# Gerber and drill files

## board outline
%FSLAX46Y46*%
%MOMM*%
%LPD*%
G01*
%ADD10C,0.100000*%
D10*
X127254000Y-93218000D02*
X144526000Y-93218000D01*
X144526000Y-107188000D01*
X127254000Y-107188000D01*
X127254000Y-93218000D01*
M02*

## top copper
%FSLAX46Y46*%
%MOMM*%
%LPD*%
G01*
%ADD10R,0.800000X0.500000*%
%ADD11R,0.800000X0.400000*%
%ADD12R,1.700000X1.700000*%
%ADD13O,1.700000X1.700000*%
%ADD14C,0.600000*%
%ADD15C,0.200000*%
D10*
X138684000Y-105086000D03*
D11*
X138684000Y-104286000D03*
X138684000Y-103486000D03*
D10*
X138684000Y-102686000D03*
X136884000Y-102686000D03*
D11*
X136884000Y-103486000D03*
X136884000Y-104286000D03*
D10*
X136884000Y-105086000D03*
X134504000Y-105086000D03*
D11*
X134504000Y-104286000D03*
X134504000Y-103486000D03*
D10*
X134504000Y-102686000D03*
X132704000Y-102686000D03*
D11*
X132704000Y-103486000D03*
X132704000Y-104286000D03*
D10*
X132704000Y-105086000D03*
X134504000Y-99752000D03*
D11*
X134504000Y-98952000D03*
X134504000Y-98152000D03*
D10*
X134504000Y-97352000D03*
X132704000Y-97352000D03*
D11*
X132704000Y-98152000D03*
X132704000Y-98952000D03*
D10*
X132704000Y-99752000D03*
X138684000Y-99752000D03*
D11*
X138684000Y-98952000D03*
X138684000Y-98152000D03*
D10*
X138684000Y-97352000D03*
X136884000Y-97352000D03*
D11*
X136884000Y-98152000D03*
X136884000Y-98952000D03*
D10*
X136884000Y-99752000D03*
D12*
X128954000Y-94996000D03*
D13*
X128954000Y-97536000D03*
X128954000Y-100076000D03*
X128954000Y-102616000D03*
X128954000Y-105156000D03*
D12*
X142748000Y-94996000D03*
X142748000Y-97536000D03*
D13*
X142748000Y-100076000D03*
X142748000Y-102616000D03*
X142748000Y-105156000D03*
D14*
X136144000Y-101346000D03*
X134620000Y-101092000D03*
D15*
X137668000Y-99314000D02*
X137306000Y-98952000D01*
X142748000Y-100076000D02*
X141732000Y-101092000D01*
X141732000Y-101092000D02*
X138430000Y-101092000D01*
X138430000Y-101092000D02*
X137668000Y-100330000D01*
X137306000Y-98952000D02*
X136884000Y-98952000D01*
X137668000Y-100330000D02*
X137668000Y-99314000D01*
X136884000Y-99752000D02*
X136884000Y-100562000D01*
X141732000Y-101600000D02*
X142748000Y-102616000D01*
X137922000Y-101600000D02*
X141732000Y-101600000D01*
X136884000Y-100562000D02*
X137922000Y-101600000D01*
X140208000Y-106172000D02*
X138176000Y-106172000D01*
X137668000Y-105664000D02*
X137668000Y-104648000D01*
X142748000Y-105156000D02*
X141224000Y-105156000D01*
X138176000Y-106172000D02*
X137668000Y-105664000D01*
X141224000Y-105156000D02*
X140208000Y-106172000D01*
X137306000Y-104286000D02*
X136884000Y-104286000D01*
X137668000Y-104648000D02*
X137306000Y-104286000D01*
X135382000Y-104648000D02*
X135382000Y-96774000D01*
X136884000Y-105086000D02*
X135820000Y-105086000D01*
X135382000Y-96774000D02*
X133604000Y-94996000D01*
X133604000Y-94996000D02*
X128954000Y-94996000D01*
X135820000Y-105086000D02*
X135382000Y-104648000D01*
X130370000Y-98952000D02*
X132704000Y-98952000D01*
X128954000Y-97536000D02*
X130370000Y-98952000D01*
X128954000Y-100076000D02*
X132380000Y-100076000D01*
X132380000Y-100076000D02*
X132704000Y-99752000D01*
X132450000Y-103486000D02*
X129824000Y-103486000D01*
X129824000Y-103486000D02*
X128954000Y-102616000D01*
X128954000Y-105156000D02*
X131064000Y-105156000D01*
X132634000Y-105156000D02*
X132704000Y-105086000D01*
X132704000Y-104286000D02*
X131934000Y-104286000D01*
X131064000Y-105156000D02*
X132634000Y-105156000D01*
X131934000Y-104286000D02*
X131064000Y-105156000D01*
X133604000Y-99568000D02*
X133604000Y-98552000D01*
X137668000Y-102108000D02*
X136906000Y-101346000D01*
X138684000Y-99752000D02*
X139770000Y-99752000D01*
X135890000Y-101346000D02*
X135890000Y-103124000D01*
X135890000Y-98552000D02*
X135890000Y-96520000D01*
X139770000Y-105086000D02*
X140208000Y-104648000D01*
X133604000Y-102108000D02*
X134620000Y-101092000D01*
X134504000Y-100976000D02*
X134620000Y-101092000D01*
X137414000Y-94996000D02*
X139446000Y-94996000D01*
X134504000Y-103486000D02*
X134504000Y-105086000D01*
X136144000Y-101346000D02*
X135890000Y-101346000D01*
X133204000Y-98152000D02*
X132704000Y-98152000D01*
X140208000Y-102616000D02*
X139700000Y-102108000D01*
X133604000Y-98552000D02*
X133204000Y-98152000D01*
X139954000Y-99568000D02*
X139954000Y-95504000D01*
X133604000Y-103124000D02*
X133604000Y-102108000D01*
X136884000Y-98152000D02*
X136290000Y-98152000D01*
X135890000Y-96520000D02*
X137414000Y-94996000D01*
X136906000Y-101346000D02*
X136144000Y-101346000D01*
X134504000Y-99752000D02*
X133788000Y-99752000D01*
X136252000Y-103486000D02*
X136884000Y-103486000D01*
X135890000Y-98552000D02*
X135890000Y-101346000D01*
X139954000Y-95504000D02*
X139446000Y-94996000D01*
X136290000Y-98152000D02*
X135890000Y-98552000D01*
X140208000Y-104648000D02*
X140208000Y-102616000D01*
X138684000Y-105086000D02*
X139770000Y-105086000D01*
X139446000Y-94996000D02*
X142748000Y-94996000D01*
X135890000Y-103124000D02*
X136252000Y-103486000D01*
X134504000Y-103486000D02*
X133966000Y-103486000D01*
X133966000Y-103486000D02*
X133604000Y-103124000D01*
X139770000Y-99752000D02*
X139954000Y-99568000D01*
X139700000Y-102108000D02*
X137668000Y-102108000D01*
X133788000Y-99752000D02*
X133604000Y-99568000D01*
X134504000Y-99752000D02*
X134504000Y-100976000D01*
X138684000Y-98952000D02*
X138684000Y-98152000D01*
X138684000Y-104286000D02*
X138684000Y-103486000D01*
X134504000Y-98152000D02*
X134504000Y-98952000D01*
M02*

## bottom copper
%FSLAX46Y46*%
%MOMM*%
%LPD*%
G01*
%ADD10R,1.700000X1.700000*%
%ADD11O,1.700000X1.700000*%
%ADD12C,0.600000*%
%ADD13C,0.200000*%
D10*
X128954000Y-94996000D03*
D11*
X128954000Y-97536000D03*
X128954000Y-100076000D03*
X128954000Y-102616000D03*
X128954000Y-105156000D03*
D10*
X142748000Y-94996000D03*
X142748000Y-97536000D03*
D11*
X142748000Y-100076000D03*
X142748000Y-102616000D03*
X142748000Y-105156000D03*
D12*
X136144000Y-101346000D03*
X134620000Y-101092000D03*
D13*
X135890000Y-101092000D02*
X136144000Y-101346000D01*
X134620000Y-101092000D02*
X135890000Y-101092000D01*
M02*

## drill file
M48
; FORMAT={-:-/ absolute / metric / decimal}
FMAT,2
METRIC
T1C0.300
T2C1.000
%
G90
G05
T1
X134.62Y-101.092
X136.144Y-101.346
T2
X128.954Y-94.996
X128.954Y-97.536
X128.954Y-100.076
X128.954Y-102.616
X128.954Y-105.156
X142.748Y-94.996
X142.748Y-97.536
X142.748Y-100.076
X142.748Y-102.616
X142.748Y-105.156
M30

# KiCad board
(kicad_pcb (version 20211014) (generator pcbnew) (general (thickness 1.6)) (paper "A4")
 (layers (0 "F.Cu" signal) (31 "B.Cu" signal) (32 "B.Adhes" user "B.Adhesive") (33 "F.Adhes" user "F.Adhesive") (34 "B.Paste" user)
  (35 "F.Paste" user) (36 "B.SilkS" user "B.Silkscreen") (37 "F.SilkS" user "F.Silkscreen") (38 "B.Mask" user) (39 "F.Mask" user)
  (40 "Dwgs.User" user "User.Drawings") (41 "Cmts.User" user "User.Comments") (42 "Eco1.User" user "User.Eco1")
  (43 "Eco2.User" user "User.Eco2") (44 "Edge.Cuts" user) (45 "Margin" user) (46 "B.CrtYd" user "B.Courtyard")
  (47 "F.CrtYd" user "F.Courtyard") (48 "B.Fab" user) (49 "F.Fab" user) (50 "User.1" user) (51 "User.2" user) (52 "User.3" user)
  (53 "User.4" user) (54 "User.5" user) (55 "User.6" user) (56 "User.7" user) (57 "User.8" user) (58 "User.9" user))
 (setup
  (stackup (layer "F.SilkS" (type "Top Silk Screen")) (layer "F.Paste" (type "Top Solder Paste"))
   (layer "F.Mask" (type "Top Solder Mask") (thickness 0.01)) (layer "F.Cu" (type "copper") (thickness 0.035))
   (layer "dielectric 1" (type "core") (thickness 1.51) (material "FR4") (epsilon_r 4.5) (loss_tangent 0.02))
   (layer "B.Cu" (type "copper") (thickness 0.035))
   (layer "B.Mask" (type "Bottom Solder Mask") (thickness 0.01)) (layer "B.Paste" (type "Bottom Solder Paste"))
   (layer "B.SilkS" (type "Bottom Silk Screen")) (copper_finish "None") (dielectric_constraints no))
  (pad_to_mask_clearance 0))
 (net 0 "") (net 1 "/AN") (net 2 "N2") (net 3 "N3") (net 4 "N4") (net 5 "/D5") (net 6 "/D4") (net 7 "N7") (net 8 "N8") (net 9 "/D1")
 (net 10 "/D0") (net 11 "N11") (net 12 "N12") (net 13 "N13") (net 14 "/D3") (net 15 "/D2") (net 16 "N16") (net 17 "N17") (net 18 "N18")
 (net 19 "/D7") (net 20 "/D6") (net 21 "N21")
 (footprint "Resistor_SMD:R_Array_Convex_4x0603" (layer "F.Cu") (at 137.784 103.886 180)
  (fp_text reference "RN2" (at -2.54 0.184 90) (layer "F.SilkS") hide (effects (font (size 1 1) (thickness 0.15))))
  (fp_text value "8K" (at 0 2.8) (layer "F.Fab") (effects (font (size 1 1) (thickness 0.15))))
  (pad "1" smd rect (at -0.9 -1.2 180) (size 0.8 0.5) (layers "F.Cu" "F.Paste" "F.Mask") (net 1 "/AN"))
  (pad "2" smd rect (at -0.9 -0.4 180) (size 0.8 0.4) (layers "F.Cu" "F.Paste" "F.Mask") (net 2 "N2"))
  (pad "3" smd rect (at -0.9 0.4 180) (size 0.8 0.4) (layers "F.Cu" "F.Paste" "F.Mask") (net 2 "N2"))
  (pad "4" smd rect (at -0.9 1.2 180) (size 0.8 0.5) (layers "F.Cu" "F.Paste" "F.Mask") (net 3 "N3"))
  (pad "5" smd rect (at 0.9 1.2 180) (size 0.8 0.5) (layers "F.Cu" "F.Paste" "F.Mask") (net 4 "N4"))
  (pad "6" smd rect (at 0.9 0.4 180) (size 0.8 0.4) (layers "F.Cu" "F.Paste" "F.Mask") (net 1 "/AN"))
  (pad "7" smd rect (at 0.9 -0.4 180) (size 0.8 0.4) (layers "F.Cu" "F.Paste" "F.Mask") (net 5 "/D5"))
  (pad "8" smd rect (at 0.9 -1.2 180) (size 0.8 0.5) (layers "F.Cu" "F.Paste" "F.Mask") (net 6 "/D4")))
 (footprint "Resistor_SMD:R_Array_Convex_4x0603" (layer "F.Cu") (at 133.604 103.886 180)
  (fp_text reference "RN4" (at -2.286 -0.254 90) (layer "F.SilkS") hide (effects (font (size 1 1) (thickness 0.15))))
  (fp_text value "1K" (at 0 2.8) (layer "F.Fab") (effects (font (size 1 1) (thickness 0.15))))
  (pad "1" smd rect (at -0.9 -1.2 180) (size 0.8 0.5) (layers "F.Cu" "F.Paste" "F.Mask") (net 1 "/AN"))
  (pad "2" smd rect (at -0.9 -0.4 180) (size 0.8 0.4) (layers "F.Cu" "F.Paste" "F.Mask") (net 1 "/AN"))
  (pad "3" smd rect (at -0.9 0.4 180) (size 0.8 0.4) (layers "F.Cu" "F.Paste" "F.Mask") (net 1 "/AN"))
  (pad "4" smd rect (at -0.9 1.2 180) (size 0.8 0.5) (layers "F.Cu" "F.Paste" "F.Mask") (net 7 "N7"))
  (pad "5" smd rect (at 0.9 1.2 180) (size 0.8 0.5) (layers "F.Cu" "F.Paste" "F.Mask") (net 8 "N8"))
  (pad "6" smd rect (at 0.9 0.4 180) (size 0.8 0.4) (layers "F.Cu" "F.Paste" "F.Mask") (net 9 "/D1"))
  (pad "7" smd rect (at 0.9 -0.4 180) (size 0.8 0.4) (layers "F.Cu" "F.Paste" "F.Mask") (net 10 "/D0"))
  (pad "8" smd rect (at 0.9 -1.2 180) (size 0.8 0.5) (layers "F.Cu" "F.Paste" "F.Mask") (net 10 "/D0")))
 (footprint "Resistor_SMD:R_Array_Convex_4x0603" (layer "F.Cu") (at 133.604 98.552 180)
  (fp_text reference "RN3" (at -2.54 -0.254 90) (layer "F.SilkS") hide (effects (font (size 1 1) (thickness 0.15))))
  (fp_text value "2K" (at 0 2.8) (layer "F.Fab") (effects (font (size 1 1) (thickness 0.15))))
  (pad "1" smd rect (at -0.9 -1.2 180) (size 0.8 0.5) (layers "F.Cu" "F.Paste" "F.Mask") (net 1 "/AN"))
  (pad "2" smd rect (at -0.9 -0.4 180) (size 0.8 0.4) (layers "F.Cu" "F.Paste" "F.Mask") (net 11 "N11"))
  (pad "3" smd rect (at -0.9 0.4 180) (size 0.8 0.4) (layers "F.Cu" "F.Paste" "F.Mask") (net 11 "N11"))
  (pad "4" smd rect (at -0.9 1.2 180) (size 0.8 0.5) (layers "F.Cu" "F.Paste" "F.Mask") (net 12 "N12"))
  (pad "5" smd rect (at 0.9 1.2 180) (size 0.8 0.5) (layers "F.Cu" "F.Paste" "F.Mask") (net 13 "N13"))
  (pad "6" smd rect (at 0.9 0.4 180) (size 0.8 0.4) (layers "F.Cu" "F.Paste" "F.Mask") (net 1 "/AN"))
  (pad "7" smd rect (at 0.9 -0.4 180) (size 0.8 0.4) (layers "F.Cu" "F.Paste" "F.Mask") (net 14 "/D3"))
  (pad "8" smd rect (at 0.9 -1.2 180) (size 0.8 0.5) (layers "F.Cu" "F.Paste" "F.Mask") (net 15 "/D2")))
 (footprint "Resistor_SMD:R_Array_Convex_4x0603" (layer "F.Cu") (at 137.784 98.552 180)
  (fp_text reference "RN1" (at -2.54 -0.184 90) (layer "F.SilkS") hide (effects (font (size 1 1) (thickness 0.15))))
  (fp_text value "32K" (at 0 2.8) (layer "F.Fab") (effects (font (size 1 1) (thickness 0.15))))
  (pad "1" smd rect (at -0.9 -1.2 180) (size 0.8 0.5) (layers "F.Cu" "F.Paste" "F.Mask") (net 1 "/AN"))
  (pad "2" smd rect (at -0.9 -0.4 180) (size 0.8 0.4) (layers "F.Cu" "F.Paste" "F.Mask") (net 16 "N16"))
  (pad "3" smd rect (at -0.9 0.4 180) (size 0.8 0.4) (layers "F.Cu" "F.Paste" "F.Mask") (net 16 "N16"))
  (pad "4" smd rect (at -0.9 1.2 180) (size 0.8 0.5) (layers "F.Cu" "F.Paste" "F.Mask") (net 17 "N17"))
  (pad "5" smd rect (at 0.9 1.2 180) (size 0.8 0.5) (layers "F.Cu" "F.Paste" "F.Mask") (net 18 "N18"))
  (pad "6" smd rect (at 0.9 0.4 180) (size 0.8 0.4) (layers "F.Cu" "F.Paste" "F.Mask") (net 1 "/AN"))
  (pad "7" smd rect (at 0.9 -0.4 180) (size 0.8 0.4) (layers "F.Cu" "F.Paste" "F.Mask") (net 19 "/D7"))
  (pad "8" smd rect (at 0.9 -1.2 180) (size 0.8 0.5) (layers "F.Cu" "F.Paste" "F.Mask") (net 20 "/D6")))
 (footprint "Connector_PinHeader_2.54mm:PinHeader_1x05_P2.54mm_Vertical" (layer "B.Cu") (at 128.954 94.996 180)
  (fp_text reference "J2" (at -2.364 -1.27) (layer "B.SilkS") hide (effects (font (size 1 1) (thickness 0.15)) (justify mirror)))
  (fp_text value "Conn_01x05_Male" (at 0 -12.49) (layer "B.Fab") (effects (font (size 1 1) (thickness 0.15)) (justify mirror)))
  (pad "1" thru_hole rect (at 0 0 180) (size 1.7 1.7) (drill 1) (layers *.Cu *.Mask) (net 6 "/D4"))
  (pad "2" thru_hole oval (at 0 -2.54 180) (size 1.7 1.7) (drill 1) (layers *.Cu *.Mask) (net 14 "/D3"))
  (pad "3" thru_hole oval (at 0 -5.08 180) (size 1.7 1.7) (drill 1) (layers *.Cu *.Mask) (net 15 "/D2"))
  (pad "4" thru_hole oval (at 0 -7.62 180) (size 1.7 1.7) (drill 1) (layers *.Cu *.Mask) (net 9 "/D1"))
  (pad "5" thru_hole oval (at 0 -10.16 180) (size 1.7 1.7) (drill 1) (layers *.Cu *.Mask) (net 10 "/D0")))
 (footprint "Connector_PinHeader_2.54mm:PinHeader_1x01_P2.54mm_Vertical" (layer "B.Cu") (at 142.748 94.996 180)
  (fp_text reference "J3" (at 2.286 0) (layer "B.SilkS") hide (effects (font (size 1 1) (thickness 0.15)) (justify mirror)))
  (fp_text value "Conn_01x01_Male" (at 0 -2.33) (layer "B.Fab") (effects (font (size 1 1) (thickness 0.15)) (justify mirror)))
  (pad "1" thru_hole rect (at 0 0 180) (size 1.7 1.7) (drill 1) (layers *.Cu *.Mask) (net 1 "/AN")))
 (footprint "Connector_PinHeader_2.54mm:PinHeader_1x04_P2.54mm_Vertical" (layer "B.Cu") (at 142.748 97.536 180)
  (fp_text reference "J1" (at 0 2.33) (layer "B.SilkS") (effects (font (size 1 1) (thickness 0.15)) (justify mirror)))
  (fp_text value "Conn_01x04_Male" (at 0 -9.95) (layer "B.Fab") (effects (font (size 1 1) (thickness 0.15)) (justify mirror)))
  (pad "1" thru_hole rect (at 0 0 180) (size 1.7 1.7) (drill 1) (layers *.Cu *.Mask) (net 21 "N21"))
  (pad "2" thru_hole oval (at 0 -2.54 180) (size 1.7 1.7) (drill 1) (layers *.Cu *.Mask) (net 19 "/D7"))
  (pad "3" thru_hole oval (at 0 -5.08 180) (size 1.7 1.7) (drill 1) (layers *.Cu *.Mask) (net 20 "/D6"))
  (pad "4" thru_hole oval (at 0 -7.62 180) (size 1.7 1.7) (drill 1) (layers *.Cu *.Mask) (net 5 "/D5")))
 (gr_rect (start 127.254 93.218) (end 144.526 107.188) (layer "Edge.Cuts") (width 0.1) (fill none))
 (segment (start 137.668 99.314) (end 137.306 98.952) (width 0.2) (layer "F.Cu") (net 19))
 (segment (start 142.748 100.076) (end 141.732 101.092) (width 0.2) (layer "F.Cu") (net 19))
 (segment (start 141.732 101.092) (end 138.43 101.092) (width 0.2) (layer "F.Cu") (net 19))
 (segment (start 138.43 101.092) (end 137.668 100.33) (width 0.2) (layer "F.Cu") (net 19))
 (segment (start 137.306 98.952) (end 136.884 98.952) (width 0.2) (layer "F.Cu") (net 19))
 (segment (start 137.668 100.33) (end 137.668 99.314) (width 0.2) (layer "F.Cu") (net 19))
 (segment (start 136.884 99.752) (end 136.884 100.562) (width 0.2) (layer "F.Cu") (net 20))
 (segment (start 141.732 101.6) (end 142.748 102.616) (width 0.2) (layer "F.Cu") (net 20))
 (segment (start 137.922 101.6) (end 141.732 101.6) (width 0.2) (layer "F.Cu") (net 20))
 (segment (start 136.884 100.562) (end 137.922 101.6) (width 0.2) (layer "F.Cu") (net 20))
 (segment (start 140.208 106.172) (end 138.176 106.172) (width 0.2) (layer "F.Cu") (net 5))
 (segment (start 137.668 105.664) (end 137.668 104.648) (width 0.2) (layer "F.Cu") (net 5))
 (segment (start 142.748 105.156) (end 141.224 105.156) (width 0.2) (layer "F.Cu") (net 5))
 (segment (start 138.176 106.172) (end 137.668 105.664) (width 0.2) (layer "F.Cu") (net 5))
 (segment (start 141.224 105.156) (end 140.208 106.172) (width 0.2) (layer "F.Cu") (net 5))
 (segment (start 137.306 104.286) (end 136.884 104.286) (width 0.2) (layer "F.Cu") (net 5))
 (segment (start 137.668 104.648) (end 137.306 104.286) (width 0.2) (layer "F.Cu") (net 5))
 (segment (start 135.382 104.648) (end 135.382 96.774) (width 0.2) (layer "F.Cu") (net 6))
 (segment (start 136.884 105.086) (end 135.82 105.086) (width 0.2) (layer "F.Cu") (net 6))
 (segment (start 135.382 96.774) (end 133.604 94.996) (width 0.2) (layer "F.Cu") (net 6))
 (segment (start 133.604 94.996) (end 128.954 94.996) (width 0.2) (layer "F.Cu") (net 6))
 (segment (start 135.82 105.086) (end 135.382 104.648) (width 0.2) (layer "F.Cu") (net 6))
 (segment (start 130.37 98.952) (end 132.704 98.952) (width 0.2) (layer "F.Cu") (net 14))
 (segment (start 128.954 97.536) (end 130.37 98.952) (width 0.2) (layer "F.Cu") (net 14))
 (segment (start 128.954 100.076) (end 132.38 100.076) (width 0.2) (layer "F.Cu") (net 15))
 (segment (start 132.38 100.076) (end 132.704 99.752) (width 0.2) (layer "F.Cu") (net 15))
 (segment (start 132.45 103.486) (end 129.824 103.486) (width 0.2) (layer "F.Cu") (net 9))
 (segment (start 129.824 103.486) (end 128.954 102.616) (width 0.2) (layer "F.Cu") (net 9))
 (segment (start 128.954 105.156) (end 131.064 105.156) (width 0.2) (layer "F.Cu") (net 10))
 (segment (start 132.634 105.156) (end 132.704 105.086) (width 0.2) (layer "F.Cu") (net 10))
 (segment (start 132.704 104.286) (end 131.934 104.286) (width 0.2) (layer "F.Cu") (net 10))
 (segment (start 131.064 105.156) (end 132.634 105.156) (width 0.2) (layer "F.Cu") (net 10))
 (segment (start 131.934 104.286) (end 131.064 105.156) (width 0.2) (layer "F.Cu") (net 10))
 (segment (start 133.604 99.568) (end 133.604 98.552) (width 0.2) (layer "F.Cu") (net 1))
 (segment (start 137.668 102.108) (end 136.906 101.346) (width 0.2) (layer "F.Cu") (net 1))
 (segment (start 138.684 99.752) (end 139.77 99.752) (width 0.2) (layer "F.Cu") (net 1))
 (segment (start 135.89 101.346) (end 135.89 103.124) (width 0.2) (layer "F.Cu") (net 1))
 (segment (start 135.89 98.552) (end 135.89 96.52) (width 0.2) (layer "F.Cu") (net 1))
 (segment (start 139.77 105.086) (end 140.208 104.648) (width 0.2) (layer "F.Cu") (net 1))
 (segment (start 133.604 102.108) (end 134.62 101.092) (width 0.2) (layer "F.Cu") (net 1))
 (segment (start 134.504 100.976) (end 134.62 101.092) (width 0.2) (layer "F.Cu") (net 1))
 (segment (start 137.414 94.996) (end 139.446 94.996) (width 0.2) (layer "F.Cu") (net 1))
 (segment (start 134.504 103.486) (end 134.504 105.086) (width 0.2) (layer "F.Cu") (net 1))
 (segment (start 136.144 101.346) (end 135.89 101.346) (width 0.2) (layer "F.Cu") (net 1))
 (segment (start 133.204 98.152) (end 132.704 98.152) (width 0.2) (layer "F.Cu") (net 1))
 (segment (start 140.208 102.616) (end 139.7 102.108) (width 0.2) (layer "F.Cu") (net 1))
 (segment (start 133.604 98.552) (end 133.204 98.152) (width 0.2) (layer "F.Cu") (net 1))
 (segment (start 139.954 99.568) (end 139.954 95.504) (width 0.2) (layer "F.Cu") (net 1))
 (segment (start 133.604 103.124) (end 133.604 102.108) (width 0.2) (layer "F.Cu") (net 1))
 (segment (start 136.884 98.152) (end 136.29 98.152) (width 0.2) (layer "F.Cu") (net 1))
 (segment (start 135.89 96.52) (end 137.414 94.996) (width 0.2) (layer "F.Cu") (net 1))
 (segment (start 136.906 101.346) (end 136.144 101.346) (width 0.2) (layer "F.Cu") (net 1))
 (segment (start 134.504 99.752) (end 133.788 99.752) (width 0.2) (layer "F.Cu") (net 1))
 (segment (start 136.252 103.486) (end 136.884 103.486) (width 0.2) (layer "F.Cu") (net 1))
 (segment (start 135.89 98.552) (end 135.89 101.346) (width 0.2) (layer "F.Cu") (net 1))
 (segment (start 139.954 95.504) (end 139.446 94.996) (width 0.2) (layer "F.Cu") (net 1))
 (segment (start 136.29 98.152) (end 135.89 98.552) (width 0.2) (layer "F.Cu") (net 1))
 (segment (start 140.208 104.648) (end 140.208 102.616) (width 0.2) (layer "F.Cu") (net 1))
 (segment (start 138.684 105.086) (end 139.77 105.086) (width 0.2) (layer "F.Cu") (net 1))
 (segment (start 139.446 94.996) (end 142.748 94.996) (width 0.2) (layer "F.Cu") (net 1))
 (segment (start 135.89 103.124) (end 136.252 103.486) (width 0.2) (layer "F.Cu") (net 1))
 (segment (start 134.504 103.486) (end 133.966 103.486) (width 0.2) (layer "F.Cu") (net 1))
 (segment (start 133.966 103.486) (end 133.604 103.124) (width 0.2) (layer "F.Cu") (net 1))
 (segment (start 139.77 99.752) (end 139.954 99.568) (width 0.2) (layer "F.Cu") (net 1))
 (segment (start 139.7 102.108) (end 137.668 102.108) (width 0.2) (layer "F.Cu") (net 1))
 (segment (start 133.788 99.752) (end 133.604 99.568) (width 0.2) (layer "F.Cu") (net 1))
 (segment (start 134.504 99.752) (end 134.504 100.976) (width 0.2) (layer "F.Cu") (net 1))
 (via (at 136.144 101.346) (size 0.6) (drill 0.3) (layers "F.Cu" "B.Cu") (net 1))
 (via (at 134.62 101.092) (size 0.6) (drill 0.3) (layers "F.Cu" "B.Cu") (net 1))
 (segment (start 135.89 101.092) (end 136.144 101.346) (width 0.2) (layer "B.Cu") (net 1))
 (segment (start 134.62 101.092) (end 135.89 101.092) (width 0.2) (layer "B.Cu") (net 1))
 (segment (start 138.684 98.952) (end 138.684 98.152) (width 0.2) (layer "F.Cu") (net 16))
 (segment (start 138.684 104.286) (end 138.684 103.486) (width 0.2) (layer "F.Cu") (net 2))
 (segment (start 134.504 98.152) (end 134.504 98.952) (width 0.2) (layer "F.Cu") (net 11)))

